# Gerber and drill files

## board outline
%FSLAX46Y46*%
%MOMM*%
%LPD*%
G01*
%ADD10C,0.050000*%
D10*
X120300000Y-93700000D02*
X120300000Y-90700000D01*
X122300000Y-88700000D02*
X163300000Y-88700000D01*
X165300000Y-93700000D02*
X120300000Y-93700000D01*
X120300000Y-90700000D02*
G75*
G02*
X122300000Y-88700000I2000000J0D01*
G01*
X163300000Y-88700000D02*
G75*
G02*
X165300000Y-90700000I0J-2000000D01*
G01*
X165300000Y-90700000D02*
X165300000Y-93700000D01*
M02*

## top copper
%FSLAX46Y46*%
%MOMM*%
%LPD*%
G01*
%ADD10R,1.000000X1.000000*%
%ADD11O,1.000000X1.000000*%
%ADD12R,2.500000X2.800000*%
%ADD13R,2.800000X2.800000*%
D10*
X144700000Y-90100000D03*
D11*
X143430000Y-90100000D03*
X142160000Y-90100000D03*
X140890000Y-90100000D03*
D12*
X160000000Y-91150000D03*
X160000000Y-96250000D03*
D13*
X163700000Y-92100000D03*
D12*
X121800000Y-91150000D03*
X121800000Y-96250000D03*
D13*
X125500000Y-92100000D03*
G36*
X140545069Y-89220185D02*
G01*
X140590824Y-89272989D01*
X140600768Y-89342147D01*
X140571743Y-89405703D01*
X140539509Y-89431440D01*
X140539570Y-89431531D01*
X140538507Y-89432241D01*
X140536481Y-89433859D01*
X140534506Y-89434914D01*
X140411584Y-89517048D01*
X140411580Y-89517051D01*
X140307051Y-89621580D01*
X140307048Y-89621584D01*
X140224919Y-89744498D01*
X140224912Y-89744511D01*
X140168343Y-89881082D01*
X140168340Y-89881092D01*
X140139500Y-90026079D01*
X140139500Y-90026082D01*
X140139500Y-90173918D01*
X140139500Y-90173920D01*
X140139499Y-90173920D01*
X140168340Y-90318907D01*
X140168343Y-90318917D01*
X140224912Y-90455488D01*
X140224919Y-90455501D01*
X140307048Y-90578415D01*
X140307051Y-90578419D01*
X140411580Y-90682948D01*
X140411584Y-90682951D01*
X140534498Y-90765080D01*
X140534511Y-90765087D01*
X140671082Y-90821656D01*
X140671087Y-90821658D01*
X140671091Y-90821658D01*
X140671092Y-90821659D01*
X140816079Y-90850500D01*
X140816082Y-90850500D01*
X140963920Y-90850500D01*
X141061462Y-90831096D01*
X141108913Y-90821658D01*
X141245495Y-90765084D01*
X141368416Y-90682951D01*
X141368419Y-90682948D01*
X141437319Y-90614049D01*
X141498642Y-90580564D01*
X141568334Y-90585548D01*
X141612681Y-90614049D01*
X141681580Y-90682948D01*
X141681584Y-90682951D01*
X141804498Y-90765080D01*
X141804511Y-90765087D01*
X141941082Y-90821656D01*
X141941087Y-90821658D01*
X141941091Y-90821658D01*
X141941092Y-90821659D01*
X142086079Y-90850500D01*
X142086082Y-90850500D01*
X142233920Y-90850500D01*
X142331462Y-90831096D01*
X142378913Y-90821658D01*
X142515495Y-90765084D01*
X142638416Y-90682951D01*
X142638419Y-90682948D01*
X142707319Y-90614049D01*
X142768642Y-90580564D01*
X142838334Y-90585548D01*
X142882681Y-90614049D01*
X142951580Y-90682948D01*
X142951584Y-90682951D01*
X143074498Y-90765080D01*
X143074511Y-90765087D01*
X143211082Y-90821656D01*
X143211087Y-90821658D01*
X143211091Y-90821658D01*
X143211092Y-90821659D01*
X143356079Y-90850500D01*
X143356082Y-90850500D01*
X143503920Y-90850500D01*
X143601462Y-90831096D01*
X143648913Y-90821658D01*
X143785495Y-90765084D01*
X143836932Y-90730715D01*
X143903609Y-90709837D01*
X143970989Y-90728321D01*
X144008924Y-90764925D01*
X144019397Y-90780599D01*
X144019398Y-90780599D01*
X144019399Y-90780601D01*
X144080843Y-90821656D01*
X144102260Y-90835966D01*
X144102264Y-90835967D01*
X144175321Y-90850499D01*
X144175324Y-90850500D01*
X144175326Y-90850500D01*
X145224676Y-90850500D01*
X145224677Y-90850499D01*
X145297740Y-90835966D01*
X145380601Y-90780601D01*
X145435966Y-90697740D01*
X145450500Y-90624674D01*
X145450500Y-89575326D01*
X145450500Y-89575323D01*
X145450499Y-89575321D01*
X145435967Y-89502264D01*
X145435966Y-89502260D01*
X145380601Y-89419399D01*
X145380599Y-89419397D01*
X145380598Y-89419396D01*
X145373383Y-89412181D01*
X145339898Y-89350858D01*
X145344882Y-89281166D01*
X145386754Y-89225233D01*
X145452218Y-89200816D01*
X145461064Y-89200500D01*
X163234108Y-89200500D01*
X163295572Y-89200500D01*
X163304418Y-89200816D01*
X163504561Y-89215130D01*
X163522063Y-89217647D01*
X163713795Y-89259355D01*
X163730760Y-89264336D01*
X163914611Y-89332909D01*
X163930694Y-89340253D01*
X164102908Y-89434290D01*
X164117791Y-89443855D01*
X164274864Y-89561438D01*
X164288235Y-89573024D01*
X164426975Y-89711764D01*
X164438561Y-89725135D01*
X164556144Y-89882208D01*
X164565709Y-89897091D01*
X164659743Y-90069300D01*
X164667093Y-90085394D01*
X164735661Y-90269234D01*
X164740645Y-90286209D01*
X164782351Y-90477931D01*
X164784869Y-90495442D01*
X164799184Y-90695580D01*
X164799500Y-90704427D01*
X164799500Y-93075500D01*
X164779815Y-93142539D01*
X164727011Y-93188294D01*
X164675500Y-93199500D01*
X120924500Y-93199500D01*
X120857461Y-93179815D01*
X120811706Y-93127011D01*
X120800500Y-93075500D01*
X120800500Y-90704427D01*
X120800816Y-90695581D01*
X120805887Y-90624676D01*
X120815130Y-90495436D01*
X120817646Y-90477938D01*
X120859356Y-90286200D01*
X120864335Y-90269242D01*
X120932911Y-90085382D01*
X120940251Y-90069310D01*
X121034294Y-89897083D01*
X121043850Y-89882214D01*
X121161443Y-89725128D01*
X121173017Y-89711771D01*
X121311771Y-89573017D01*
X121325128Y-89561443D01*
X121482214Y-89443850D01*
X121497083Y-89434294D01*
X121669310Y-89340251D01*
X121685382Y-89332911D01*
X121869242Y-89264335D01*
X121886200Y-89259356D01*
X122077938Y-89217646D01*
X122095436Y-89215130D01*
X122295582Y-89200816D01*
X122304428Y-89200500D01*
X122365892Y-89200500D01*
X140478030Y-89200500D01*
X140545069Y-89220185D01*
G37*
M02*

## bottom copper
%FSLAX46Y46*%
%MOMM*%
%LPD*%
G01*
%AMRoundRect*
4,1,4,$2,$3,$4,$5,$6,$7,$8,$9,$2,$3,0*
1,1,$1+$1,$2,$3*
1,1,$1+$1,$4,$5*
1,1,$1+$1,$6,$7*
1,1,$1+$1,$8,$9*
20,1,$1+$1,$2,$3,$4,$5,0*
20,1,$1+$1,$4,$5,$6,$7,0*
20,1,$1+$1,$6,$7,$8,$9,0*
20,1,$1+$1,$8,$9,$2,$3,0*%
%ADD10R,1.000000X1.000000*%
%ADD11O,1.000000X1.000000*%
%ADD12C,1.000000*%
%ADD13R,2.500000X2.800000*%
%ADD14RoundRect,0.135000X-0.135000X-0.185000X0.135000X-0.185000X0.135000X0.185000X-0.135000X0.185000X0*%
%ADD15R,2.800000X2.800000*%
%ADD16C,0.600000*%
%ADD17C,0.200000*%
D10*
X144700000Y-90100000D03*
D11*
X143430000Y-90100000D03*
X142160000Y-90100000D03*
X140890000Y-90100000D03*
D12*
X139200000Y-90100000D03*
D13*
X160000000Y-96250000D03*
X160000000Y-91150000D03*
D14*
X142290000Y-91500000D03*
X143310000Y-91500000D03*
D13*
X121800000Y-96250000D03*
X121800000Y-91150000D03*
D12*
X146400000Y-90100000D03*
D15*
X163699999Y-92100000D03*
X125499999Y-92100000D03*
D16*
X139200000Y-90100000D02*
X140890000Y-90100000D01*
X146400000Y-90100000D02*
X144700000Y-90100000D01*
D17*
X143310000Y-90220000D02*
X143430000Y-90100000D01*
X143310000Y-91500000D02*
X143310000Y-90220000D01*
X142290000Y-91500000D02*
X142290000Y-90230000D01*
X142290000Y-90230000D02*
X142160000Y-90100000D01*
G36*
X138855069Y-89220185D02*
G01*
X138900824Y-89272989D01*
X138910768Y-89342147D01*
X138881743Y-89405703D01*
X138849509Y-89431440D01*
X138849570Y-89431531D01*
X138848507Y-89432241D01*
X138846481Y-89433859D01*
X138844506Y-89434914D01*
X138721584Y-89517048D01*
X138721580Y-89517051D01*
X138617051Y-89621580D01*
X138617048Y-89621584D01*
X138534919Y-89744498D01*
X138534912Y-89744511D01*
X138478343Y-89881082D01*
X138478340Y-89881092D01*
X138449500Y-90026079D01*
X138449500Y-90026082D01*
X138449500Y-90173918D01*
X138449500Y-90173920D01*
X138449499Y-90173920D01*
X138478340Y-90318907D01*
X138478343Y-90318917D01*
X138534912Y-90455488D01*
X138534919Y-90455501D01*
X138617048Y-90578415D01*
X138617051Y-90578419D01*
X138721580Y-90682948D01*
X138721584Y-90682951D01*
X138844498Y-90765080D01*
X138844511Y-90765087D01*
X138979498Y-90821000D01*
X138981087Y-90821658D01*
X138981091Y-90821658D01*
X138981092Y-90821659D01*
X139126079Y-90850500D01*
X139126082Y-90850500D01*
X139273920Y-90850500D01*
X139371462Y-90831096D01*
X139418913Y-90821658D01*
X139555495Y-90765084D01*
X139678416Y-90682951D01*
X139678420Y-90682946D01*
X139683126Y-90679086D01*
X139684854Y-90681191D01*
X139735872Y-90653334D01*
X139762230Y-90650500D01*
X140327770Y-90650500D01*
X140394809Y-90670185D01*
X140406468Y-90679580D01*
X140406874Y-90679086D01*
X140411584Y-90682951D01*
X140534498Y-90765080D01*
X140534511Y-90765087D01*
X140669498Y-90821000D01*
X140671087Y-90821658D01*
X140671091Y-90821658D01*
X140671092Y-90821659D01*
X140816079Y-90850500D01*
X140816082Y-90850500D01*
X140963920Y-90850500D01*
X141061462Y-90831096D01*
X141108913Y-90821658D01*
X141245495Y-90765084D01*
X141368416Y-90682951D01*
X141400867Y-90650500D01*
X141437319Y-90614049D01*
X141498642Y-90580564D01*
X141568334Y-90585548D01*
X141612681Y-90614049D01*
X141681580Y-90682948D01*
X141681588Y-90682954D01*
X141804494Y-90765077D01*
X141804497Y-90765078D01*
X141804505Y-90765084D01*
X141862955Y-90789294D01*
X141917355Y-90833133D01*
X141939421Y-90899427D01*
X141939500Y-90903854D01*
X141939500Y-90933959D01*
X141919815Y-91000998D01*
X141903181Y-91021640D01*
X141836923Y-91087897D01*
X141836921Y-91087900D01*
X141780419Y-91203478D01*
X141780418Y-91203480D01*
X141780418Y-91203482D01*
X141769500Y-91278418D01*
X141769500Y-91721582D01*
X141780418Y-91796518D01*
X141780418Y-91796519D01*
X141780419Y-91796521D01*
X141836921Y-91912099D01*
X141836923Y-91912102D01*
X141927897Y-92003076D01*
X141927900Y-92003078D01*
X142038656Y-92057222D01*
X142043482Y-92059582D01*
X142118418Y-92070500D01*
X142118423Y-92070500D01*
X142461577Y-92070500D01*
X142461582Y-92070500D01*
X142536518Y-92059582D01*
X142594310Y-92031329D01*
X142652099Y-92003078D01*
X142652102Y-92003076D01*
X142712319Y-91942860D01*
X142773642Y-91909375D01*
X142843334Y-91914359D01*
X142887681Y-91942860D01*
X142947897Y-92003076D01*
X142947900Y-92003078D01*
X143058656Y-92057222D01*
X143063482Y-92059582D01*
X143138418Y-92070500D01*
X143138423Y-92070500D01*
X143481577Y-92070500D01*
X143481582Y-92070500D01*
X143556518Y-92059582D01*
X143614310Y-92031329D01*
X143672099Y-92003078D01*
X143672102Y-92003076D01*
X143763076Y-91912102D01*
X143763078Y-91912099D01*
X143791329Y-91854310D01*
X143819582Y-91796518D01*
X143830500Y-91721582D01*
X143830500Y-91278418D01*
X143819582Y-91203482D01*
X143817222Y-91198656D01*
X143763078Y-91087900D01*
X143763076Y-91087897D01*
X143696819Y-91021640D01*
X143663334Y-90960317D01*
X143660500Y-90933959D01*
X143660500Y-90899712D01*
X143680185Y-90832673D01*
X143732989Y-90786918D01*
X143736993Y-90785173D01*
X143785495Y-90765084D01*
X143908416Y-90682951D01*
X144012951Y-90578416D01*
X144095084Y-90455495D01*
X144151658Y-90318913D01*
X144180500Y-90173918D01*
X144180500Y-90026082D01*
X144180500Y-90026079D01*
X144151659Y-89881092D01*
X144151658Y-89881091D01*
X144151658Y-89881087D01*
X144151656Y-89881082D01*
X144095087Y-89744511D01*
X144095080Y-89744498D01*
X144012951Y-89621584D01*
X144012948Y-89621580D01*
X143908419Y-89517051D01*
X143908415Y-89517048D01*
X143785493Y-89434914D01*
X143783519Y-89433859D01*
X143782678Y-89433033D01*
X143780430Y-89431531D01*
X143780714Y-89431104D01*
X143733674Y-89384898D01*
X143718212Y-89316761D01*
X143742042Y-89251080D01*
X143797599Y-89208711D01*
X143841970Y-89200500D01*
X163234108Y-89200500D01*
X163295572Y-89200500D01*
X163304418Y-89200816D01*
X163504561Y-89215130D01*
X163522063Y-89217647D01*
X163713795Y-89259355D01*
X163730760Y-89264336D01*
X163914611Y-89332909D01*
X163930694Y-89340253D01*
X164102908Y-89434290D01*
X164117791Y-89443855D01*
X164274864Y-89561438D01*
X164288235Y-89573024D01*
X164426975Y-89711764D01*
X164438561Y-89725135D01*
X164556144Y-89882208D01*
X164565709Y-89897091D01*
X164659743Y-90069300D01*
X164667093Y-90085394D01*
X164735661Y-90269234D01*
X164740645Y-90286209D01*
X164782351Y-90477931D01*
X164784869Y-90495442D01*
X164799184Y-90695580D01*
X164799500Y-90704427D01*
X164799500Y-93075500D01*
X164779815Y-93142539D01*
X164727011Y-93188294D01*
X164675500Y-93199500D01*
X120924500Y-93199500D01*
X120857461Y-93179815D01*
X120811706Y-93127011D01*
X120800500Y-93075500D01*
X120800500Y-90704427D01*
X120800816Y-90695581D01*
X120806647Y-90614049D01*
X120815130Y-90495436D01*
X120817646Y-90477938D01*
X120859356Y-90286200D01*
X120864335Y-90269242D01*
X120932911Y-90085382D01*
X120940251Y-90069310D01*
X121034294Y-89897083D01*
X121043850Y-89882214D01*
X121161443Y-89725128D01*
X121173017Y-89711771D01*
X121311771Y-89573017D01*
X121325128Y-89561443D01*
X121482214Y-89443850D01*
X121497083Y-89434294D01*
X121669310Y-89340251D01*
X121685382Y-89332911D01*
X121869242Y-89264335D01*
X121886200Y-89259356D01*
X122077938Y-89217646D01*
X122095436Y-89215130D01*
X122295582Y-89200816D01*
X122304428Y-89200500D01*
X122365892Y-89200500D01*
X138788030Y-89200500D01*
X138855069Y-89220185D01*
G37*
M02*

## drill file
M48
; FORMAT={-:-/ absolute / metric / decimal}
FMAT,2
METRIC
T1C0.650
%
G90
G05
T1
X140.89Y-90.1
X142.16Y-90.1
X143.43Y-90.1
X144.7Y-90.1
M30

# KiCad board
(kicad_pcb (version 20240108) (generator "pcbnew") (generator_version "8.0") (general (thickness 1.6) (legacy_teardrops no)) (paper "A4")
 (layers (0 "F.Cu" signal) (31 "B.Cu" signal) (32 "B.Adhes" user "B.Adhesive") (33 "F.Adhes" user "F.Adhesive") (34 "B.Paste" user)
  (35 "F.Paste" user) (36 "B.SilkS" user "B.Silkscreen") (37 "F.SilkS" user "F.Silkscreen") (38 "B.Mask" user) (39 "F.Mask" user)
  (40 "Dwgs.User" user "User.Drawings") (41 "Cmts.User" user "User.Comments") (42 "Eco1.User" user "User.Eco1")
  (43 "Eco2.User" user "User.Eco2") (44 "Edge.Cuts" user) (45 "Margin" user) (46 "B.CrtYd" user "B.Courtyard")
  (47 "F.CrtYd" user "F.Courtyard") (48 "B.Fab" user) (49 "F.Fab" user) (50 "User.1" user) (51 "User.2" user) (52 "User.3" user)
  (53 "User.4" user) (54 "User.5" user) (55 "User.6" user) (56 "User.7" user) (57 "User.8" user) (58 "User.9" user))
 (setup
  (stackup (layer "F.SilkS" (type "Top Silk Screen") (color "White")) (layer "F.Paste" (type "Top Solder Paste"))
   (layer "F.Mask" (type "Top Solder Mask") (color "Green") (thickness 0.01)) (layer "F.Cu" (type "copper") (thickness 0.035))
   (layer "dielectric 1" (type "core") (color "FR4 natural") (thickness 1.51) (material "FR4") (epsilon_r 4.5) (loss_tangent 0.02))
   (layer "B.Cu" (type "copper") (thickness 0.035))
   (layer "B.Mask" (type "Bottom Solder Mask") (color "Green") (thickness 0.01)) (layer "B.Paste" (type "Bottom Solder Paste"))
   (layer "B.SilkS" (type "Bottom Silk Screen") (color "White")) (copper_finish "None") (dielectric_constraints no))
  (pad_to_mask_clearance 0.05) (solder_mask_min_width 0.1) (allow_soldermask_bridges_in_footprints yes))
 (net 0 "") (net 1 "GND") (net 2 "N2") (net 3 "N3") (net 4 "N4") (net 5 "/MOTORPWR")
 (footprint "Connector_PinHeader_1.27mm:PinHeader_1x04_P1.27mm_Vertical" (layer "F.Cu") (at 144.7 90.1 -90)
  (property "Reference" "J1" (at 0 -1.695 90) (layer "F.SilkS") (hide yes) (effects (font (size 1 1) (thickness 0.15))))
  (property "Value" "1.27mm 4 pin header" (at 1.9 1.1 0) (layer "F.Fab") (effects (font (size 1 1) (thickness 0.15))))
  (pad "1" thru_hole rect (at 0 0 270) (size 1 1) (drill 0.65) (layers "*.Cu" "*.Mask") (remove_unused_layers no) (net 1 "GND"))
  (pad "2" thru_hole oval (at 0 1.27 270) (size 1 1) (drill 0.65) (layers "*.Cu" "*.Mask") (remove_unused_layers no) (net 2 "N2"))
  (pad "3" thru_hole oval (at 0 2.54 270) (size 1 1) (drill 0.65) (layers "*.Cu" "*.Mask") (remove_unused_layers no) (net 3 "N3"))
  (pad "4" thru_hole oval (at 0 3.81 270) (size 1 1) (drill 0.65) (layers "*.Cu" "*.Mask") (remove_unused_layers no) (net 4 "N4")))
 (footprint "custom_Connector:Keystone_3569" (layer "F.Cu") (at 160 93.7)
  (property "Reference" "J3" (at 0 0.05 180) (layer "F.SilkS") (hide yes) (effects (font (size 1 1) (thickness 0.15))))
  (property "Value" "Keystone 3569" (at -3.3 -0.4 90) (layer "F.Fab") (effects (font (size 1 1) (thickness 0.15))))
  (pad "1" smd rect (at 0 -2.55) (size 2.5 2.8) (layers "F.Cu" "F.Paste" "F.Mask") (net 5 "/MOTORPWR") (solder_mask_margin 0.1)
   (thermal_bridge_angle 45))
  (pad "1" smd rect (at 0 2.55) (size 2.5 2.8) (layers "F.Cu" "F.Paste" "F.Mask") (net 5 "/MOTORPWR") (solder_mask_margin 0.1)
   (thermal_bridge_angle 45)))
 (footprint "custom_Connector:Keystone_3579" (layer "F.Cu") (at 163.7 92.1)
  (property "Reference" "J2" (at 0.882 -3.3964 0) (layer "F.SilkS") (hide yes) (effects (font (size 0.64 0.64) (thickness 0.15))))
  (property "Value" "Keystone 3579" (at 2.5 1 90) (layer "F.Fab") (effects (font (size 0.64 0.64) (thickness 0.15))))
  (pad "1" smd rect (at 0 0) (size 2.8 2.8) (layers "F.Cu" "F.Paste" "F.Mask") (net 5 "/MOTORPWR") (solder_mask_margin 0.102)))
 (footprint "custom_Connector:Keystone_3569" (layer "F.Cu") (at 121.8 93.7)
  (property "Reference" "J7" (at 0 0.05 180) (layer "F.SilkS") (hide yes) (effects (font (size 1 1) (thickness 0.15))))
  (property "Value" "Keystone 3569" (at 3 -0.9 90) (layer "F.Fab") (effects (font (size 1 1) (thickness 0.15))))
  (pad "1" smd rect (at 0 -2.55) (size 2.5 2.8) (layers "F.Cu" "F.Paste" "F.Mask") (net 5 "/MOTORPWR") (solder_mask_margin 0.1)
   (thermal_bridge_angle 45))
  (pad "1" smd rect (at 0 2.55) (size 2.5 2.8) (layers "F.Cu" "F.Paste" "F.Mask") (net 5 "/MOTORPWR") (solder_mask_margin 0.1)
   (thermal_bridge_angle 45)))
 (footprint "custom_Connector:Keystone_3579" (layer "F.Cu") (at 125.5 92.1)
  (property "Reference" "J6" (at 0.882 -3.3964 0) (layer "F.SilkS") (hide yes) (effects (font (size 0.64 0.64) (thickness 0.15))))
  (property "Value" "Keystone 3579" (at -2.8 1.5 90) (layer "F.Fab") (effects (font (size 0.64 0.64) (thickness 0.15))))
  (pad "1" smd rect (at 0 0) (size 2.8 2.8) (layers "F.Cu" "F.Paste" "F.Mask") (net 5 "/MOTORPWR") (solder_mask_margin 0.102)))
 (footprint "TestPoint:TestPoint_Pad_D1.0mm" (layer "B.Cu") (at 139.2 90.1 180)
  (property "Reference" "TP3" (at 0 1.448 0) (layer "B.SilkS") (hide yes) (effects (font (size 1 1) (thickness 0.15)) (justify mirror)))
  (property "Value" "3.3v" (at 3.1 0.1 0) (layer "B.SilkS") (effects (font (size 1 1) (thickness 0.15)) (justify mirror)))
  (pad "1" smd circle (at 0 0 180) (size 1 1) (layers "B.Cu" "B.Mask") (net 4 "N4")))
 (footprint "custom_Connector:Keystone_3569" (layer "B.Cu") (at 160 93.7 180)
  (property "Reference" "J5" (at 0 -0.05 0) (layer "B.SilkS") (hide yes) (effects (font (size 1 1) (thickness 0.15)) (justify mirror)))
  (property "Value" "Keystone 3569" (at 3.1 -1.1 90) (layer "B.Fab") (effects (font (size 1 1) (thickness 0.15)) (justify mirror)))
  (pad "1" smd rect (at 0 -2.55 180) (size 2.5 2.8) (layers "B.Cu" "B.Paste" "B.Mask") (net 1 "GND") (solder_mask_margin 0.1)
   (thermal_bridge_angle 45))
  (pad "1" smd rect (at 0 2.55 180) (size 2.5 2.8) (layers "B.Cu" "B.Paste" "B.Mask") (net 1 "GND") (solder_mask_margin 0.1)
   (thermal_bridge_angle 45)))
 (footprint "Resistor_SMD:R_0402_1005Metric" (layer "B.Cu") (at 142.8 91.5)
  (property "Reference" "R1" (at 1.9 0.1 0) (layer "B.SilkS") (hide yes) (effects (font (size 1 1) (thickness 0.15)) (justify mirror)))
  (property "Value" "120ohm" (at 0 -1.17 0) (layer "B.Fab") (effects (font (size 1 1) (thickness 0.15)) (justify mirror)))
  (pad "1" smd roundrect (at -0.51 0) (size 0.54 0.64) (layers "B.Cu" "B.Paste" "B.Mask") (roundrect_rratio 0.25) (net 3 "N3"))
  (pad "2" smd roundrect (at 0.51 0) (size 0.54 0.64) (layers "B.Cu" "B.Paste" "B.Mask") (roundrect_rratio 0.25) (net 2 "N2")))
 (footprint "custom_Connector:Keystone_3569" (layer "B.Cu") (at 121.8 93.7 180)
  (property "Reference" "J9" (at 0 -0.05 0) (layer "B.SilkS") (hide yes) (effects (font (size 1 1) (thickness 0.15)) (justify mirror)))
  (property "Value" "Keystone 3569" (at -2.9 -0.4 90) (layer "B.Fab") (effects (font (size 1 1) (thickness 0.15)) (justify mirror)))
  (pad "1" smd rect (at 0 -2.55 180) (size 2.5 2.8) (layers "B.Cu" "B.Paste" "B.Mask") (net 1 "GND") (solder_mask_margin 0.1)
   (thermal_bridge_angle 45))
  (pad "1" smd rect (at 0 2.55 180) (size 2.5 2.8) (layers "B.Cu" "B.Paste" "B.Mask") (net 1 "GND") (solder_mask_margin 0.1)
   (thermal_bridge_angle 45)))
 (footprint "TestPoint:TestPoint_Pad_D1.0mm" (layer "B.Cu") (at 146.4 90.1 180)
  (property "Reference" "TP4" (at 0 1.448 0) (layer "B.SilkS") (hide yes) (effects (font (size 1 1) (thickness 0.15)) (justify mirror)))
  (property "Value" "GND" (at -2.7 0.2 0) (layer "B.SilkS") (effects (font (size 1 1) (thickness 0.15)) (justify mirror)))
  (pad "1" smd circle (at 0 0 180) (size 1 1) (layers "B.Cu" "B.Mask") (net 1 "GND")))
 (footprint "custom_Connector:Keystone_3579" (layer "B.Cu") (at 163.699999 92.1 180)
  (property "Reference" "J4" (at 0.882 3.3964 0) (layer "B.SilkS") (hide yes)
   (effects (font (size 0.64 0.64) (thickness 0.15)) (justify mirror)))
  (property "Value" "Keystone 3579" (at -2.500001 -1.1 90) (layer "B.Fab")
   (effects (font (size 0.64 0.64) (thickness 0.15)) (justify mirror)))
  (pad "1" smd rect (at 0 0 180) (size 2.8 2.8) (layers "B.Cu" "B.Paste" "B.Mask") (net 1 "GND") (solder_mask_margin 0.102)))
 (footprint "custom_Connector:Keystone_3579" (layer "B.Cu") (at 125.499999 92.1 180)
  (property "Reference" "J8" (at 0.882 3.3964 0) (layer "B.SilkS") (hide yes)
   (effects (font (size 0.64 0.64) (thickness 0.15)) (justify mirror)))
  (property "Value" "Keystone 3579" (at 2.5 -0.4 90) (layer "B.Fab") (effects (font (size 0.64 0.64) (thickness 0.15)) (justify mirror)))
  (pad "1" smd rect (at 0 0 180) (size 2.8 2.8) (layers "B.Cu" "B.Paste" "B.Mask") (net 1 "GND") (solder_mask_margin 0.102)))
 (gr_line (start 120.3 93.7) (end 120.3 90.7) (stroke (width 0.05) (type default)) (layer "Edge.Cuts"))
 (gr_line (start 122.3 88.7) (end 163.3 88.7) (stroke (width 0.05) (type default)) (layer "Edge.Cuts"))
 (gr_line (start 165.3 93.7) (end 120.3 93.7) (stroke (width 0.05) (type default)) (layer "Edge.Cuts"))
 (gr_arc (start 120.3 90.7) (mid 120.885786 89.285786) (end 122.3 88.7) (stroke (width 0.05) (type default)) (layer "Edge.Cuts"))
 (gr_arc (start 163.3 88.7) (mid 164.714214 89.285786) (end 165.3 90.7) (stroke (width 0.05) (type default)) (layer "Edge.Cuts"))
 (gr_line (start 165.3 90.7) (end 165.3 93.7) (stroke (width 0.05) (type default)) (layer "Edge.Cuts"))
 (segment (start 139.2 90.1) (end 140.89 90.1) (width 0.6) (layer "B.Cu") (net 4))
 (segment (start 146.4 90.1) (end 144.7 90.1) (width 0.6) (layer "B.Cu") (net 1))
 (segment (start 143.31 90.22) (end 143.43 90.1) (width 0.2) (layer "B.Cu") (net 2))
 (segment (start 143.31 91.5) (end 143.31 90.22) (width 0.2) (layer "B.Cu") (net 2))
 (segment (start 142.29 91.5) (end 142.29 90.23) (width 0.2) (layer "B.Cu") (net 3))
 (segment (start 142.29 90.23) (end 142.16 90.1) (width 0.2) (layer "B.Cu") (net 3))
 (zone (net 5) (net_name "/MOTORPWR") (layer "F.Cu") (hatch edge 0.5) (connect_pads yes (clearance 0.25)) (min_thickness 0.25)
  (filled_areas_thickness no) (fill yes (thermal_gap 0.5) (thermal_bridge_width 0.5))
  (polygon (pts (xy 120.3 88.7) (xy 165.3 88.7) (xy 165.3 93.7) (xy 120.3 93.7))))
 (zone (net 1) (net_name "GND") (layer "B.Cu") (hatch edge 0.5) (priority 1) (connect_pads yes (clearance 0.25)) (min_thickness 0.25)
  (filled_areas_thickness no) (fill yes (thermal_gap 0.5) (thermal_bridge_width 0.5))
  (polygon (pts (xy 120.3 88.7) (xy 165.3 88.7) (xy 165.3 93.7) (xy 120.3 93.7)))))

